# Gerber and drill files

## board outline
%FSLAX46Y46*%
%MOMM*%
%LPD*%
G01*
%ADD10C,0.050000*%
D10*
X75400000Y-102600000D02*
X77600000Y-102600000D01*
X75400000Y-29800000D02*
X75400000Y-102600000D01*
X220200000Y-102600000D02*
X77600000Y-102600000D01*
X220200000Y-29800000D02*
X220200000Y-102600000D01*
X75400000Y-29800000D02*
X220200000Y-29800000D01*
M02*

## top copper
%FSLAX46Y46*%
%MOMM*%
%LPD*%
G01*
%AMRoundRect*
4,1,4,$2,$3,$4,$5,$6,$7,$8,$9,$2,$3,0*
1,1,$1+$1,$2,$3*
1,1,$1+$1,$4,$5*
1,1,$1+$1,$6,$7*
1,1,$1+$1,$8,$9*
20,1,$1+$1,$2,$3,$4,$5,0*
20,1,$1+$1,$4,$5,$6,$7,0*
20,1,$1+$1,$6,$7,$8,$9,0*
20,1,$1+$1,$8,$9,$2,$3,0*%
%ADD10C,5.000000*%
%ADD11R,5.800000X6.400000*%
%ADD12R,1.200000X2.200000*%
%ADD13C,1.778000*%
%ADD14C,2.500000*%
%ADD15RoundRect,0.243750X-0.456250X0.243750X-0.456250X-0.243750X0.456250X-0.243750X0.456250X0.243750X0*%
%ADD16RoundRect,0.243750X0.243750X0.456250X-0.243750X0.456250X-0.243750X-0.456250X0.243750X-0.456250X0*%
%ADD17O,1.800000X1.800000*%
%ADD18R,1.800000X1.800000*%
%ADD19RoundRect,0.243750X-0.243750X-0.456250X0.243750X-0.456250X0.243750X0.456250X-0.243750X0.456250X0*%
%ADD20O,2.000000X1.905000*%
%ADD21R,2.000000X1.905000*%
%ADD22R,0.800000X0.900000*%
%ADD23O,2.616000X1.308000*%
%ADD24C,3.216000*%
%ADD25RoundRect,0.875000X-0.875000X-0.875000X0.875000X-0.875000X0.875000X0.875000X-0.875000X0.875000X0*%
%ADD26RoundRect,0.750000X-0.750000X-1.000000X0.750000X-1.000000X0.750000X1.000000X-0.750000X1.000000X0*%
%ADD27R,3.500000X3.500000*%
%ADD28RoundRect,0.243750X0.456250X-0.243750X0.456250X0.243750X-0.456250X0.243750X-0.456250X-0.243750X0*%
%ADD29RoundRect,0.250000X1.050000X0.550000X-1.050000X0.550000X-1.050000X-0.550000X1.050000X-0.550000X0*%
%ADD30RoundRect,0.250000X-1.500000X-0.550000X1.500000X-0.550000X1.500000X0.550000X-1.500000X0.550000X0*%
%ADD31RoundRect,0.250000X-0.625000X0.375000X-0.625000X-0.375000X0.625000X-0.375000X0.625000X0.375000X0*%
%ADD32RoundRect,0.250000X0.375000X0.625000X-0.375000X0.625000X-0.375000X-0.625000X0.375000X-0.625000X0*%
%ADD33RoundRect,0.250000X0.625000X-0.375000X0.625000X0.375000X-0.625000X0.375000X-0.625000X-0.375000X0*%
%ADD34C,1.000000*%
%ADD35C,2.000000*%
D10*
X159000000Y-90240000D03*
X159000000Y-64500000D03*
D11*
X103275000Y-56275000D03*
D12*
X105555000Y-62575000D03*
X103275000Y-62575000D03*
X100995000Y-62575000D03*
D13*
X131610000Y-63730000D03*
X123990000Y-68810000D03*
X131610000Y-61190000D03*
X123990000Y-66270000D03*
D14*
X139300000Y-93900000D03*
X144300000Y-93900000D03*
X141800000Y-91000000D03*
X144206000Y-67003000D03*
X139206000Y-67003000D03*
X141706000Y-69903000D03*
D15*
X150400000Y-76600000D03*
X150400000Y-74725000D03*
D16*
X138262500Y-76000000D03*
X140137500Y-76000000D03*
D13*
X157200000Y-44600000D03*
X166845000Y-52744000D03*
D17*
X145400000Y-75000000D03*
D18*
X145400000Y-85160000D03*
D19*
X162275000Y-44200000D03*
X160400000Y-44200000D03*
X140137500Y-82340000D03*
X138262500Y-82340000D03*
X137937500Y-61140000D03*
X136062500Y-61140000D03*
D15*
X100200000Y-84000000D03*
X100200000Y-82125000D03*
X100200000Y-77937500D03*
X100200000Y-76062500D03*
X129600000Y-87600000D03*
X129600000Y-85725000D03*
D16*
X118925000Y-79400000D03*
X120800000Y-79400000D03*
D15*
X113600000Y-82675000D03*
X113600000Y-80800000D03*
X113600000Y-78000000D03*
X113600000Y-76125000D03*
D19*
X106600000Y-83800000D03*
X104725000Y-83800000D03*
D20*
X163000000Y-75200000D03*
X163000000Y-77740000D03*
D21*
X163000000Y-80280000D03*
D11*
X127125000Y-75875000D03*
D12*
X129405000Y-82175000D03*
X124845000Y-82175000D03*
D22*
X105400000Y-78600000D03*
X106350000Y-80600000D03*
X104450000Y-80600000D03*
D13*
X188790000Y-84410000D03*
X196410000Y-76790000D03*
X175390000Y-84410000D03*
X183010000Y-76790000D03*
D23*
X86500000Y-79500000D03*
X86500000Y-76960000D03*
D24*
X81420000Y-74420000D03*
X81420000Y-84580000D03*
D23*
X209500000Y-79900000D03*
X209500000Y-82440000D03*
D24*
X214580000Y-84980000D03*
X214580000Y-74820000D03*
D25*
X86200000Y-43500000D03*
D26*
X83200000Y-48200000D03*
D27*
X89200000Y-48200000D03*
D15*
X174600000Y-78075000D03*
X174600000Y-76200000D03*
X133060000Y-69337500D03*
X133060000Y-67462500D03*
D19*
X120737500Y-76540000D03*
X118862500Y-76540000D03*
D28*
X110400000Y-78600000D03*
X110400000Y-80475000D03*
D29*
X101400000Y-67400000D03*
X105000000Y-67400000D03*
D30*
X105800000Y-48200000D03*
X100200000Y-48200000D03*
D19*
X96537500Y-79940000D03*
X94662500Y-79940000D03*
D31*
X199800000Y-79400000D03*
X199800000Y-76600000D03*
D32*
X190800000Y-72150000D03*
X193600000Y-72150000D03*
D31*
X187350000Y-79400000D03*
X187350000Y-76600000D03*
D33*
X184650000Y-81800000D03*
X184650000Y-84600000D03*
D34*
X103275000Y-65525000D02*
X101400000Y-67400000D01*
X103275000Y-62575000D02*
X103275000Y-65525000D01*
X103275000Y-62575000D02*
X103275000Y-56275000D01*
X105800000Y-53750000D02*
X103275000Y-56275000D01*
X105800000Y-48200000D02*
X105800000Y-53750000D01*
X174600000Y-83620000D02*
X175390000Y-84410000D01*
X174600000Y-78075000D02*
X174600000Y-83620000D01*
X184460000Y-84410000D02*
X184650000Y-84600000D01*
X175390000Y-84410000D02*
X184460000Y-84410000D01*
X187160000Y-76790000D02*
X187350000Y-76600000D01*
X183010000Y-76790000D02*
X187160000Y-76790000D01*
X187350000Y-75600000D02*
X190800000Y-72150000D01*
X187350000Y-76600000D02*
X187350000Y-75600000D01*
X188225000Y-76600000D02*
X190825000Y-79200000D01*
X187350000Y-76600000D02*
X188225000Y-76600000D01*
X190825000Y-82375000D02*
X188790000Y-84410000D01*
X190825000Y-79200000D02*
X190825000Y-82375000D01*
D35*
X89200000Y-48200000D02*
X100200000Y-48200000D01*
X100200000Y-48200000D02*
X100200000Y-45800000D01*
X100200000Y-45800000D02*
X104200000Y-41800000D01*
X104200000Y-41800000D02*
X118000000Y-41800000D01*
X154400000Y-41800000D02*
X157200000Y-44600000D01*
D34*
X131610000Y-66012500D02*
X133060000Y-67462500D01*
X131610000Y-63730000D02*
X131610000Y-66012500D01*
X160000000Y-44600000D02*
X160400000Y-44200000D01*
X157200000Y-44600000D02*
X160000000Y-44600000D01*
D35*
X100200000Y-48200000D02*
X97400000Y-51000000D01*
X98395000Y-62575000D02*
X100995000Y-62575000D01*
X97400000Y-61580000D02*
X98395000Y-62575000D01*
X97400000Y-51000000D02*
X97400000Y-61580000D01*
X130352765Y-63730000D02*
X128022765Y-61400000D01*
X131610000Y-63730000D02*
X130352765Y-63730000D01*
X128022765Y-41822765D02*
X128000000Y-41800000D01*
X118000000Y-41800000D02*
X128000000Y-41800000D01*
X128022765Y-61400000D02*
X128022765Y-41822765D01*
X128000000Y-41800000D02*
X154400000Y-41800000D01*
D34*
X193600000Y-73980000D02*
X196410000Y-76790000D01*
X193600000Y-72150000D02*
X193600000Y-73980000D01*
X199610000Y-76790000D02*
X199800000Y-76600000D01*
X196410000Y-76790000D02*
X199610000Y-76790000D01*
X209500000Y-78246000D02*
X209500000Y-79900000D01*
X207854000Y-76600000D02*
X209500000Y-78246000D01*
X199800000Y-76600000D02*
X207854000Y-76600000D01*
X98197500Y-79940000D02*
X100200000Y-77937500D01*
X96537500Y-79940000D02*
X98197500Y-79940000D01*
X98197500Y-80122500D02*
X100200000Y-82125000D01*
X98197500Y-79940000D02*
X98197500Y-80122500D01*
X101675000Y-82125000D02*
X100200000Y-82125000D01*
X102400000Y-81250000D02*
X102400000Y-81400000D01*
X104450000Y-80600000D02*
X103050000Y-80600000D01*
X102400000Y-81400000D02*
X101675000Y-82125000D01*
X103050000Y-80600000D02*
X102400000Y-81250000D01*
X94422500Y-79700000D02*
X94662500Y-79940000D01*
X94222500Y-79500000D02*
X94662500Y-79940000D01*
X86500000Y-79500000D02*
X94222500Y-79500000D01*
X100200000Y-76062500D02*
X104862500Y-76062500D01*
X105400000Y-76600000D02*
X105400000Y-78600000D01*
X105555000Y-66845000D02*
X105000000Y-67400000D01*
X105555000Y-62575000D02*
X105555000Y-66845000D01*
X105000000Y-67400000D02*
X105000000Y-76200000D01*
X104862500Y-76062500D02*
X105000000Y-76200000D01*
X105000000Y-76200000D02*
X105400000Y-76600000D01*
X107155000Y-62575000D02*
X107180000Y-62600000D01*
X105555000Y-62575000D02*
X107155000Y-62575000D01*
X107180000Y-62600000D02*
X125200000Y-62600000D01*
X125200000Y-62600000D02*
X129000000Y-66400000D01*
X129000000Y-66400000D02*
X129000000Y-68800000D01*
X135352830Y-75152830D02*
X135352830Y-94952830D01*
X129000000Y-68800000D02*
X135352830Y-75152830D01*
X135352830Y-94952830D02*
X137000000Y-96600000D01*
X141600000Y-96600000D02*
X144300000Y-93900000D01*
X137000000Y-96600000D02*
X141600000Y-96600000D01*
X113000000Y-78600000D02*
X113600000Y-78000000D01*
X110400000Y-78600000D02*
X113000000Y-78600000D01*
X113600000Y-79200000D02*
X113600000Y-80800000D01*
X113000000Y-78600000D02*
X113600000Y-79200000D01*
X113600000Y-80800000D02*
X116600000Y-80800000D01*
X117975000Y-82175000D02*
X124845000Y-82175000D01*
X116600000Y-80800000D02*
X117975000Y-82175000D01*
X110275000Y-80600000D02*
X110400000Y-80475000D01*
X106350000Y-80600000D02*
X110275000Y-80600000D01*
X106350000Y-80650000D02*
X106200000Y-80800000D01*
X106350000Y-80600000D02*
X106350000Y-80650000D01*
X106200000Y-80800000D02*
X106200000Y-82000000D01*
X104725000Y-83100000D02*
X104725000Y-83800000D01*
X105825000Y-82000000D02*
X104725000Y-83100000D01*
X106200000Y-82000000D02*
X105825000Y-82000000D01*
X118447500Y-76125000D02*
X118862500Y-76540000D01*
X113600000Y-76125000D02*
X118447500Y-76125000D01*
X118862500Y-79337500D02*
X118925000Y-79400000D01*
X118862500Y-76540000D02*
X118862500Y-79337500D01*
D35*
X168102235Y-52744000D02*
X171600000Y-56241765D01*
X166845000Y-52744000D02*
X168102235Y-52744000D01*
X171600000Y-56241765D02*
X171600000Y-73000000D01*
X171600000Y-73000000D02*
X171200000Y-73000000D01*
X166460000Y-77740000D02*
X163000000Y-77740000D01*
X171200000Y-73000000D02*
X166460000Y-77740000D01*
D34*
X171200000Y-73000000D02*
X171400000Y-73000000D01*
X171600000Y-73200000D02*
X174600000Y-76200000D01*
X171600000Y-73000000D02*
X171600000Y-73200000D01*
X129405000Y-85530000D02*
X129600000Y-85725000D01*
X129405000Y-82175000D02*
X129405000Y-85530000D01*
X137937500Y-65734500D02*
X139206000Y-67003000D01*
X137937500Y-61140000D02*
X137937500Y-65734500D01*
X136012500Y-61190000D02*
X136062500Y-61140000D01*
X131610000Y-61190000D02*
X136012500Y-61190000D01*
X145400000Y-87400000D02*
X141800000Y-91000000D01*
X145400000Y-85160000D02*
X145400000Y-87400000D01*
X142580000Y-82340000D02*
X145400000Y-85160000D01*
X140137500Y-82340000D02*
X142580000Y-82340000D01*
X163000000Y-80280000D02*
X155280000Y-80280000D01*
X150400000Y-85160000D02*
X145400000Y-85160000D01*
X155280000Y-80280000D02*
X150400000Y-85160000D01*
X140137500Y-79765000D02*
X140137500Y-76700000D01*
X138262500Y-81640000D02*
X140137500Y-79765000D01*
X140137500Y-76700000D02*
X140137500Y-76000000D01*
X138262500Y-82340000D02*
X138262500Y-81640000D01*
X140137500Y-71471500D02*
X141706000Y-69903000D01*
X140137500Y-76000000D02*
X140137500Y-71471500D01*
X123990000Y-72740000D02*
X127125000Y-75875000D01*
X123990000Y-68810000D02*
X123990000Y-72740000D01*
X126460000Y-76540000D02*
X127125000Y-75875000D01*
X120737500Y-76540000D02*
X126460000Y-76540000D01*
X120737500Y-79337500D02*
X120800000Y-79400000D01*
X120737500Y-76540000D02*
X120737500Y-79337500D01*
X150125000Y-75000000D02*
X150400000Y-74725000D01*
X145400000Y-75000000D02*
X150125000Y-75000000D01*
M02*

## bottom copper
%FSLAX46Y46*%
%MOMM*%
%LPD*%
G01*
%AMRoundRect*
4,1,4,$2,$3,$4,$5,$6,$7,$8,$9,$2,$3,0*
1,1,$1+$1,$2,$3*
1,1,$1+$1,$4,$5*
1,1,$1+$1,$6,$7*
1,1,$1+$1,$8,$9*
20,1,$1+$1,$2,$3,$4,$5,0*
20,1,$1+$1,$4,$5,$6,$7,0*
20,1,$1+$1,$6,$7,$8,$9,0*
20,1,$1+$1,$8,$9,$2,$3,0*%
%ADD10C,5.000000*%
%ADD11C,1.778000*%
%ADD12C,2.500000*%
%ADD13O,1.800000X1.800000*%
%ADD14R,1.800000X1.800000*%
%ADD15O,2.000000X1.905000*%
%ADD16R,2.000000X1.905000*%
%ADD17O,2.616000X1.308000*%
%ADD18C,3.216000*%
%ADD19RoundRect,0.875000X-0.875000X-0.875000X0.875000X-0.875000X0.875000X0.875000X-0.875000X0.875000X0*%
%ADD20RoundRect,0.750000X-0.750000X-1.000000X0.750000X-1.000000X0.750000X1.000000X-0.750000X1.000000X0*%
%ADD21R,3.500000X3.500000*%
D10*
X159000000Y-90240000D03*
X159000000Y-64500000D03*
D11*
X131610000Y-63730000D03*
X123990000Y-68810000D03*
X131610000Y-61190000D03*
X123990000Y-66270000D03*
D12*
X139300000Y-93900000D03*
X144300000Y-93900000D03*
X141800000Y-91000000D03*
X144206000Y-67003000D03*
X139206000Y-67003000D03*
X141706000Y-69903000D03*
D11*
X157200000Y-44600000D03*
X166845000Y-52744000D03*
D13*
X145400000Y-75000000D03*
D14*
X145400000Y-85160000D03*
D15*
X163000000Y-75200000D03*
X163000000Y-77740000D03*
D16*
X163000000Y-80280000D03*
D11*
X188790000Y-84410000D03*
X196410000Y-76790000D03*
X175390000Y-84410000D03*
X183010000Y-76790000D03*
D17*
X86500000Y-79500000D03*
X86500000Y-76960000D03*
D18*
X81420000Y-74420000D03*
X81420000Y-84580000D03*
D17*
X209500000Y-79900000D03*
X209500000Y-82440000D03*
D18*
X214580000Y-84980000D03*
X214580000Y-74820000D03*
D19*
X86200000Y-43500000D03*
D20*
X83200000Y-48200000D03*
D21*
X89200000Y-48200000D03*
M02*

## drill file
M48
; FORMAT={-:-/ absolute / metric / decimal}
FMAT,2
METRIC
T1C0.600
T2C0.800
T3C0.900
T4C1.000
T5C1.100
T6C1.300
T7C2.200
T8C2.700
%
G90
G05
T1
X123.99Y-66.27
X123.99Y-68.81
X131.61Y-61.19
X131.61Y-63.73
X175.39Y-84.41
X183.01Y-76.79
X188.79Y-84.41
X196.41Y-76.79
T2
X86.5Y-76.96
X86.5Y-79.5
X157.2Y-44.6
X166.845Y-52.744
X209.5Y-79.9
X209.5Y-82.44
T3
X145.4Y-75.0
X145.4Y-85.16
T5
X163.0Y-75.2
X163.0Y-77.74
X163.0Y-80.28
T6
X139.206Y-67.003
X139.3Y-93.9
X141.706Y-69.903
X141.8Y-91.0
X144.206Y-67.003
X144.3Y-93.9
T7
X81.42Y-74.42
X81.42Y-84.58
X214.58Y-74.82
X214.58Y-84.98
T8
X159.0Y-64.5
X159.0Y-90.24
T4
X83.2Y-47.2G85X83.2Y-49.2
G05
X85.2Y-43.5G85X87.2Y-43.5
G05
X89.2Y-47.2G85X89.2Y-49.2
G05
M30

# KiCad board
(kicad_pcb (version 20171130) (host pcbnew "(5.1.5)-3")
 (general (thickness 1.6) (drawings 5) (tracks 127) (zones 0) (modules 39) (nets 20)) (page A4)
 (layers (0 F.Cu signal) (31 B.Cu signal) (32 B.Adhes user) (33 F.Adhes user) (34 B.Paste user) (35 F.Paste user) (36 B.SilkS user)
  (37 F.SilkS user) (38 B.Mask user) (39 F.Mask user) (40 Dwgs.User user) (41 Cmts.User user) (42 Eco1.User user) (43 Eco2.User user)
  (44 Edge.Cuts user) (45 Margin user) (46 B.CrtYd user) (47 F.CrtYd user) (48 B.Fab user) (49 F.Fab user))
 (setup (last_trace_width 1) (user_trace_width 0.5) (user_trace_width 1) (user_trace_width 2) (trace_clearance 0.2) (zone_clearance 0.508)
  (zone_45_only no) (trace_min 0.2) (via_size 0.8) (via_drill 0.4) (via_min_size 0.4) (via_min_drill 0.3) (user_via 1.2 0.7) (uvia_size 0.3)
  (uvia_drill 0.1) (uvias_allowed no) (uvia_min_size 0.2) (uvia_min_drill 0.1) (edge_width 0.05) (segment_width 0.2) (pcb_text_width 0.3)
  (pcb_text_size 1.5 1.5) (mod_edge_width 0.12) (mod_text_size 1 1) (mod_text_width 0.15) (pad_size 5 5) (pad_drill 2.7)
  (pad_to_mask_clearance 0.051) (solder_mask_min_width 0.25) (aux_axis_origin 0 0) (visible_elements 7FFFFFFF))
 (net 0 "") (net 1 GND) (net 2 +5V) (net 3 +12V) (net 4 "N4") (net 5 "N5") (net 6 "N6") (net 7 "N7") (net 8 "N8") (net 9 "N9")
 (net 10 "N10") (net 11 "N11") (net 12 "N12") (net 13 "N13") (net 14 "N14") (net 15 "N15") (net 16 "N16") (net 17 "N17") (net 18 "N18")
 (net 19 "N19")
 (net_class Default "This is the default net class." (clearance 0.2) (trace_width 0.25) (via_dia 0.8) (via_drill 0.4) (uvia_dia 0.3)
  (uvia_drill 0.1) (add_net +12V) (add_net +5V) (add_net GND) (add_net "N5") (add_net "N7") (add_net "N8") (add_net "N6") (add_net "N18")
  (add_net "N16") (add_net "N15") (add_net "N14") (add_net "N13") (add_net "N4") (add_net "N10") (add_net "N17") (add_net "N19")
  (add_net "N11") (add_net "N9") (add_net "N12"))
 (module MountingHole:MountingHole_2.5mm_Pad (layer F.Cu) (at 159 90.24)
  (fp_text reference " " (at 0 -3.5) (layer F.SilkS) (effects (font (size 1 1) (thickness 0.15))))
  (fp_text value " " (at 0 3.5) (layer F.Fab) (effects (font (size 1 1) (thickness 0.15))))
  (pad 1 thru_hole circle (at 0 0) (size 5 5) (drill 2.7) (layers *.Cu *.Mask)))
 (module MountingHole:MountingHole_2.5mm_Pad (layer F.Cu) (at 159 64.5)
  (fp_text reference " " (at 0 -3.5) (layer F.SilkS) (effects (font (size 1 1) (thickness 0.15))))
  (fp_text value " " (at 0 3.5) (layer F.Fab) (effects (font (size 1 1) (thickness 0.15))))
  (pad 1 thru_hole circle (at 0 0) (size 5 5) (drill 2.7) (layers *.Cu *.Mask)))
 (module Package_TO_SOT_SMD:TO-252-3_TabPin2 (layer F.Cu) (at 103.275 58.375 90)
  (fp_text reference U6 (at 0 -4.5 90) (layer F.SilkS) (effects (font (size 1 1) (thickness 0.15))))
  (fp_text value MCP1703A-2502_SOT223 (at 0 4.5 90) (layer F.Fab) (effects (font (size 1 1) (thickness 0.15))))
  (pad "" smd rect (at 0.425 1.525 90) (size 3.05 2.75) (layers F.Paste))
  (pad "" smd rect (at 3.775 -1.525 90) (size 3.05 2.75) (layers F.Paste))
  (pad "" smd rect (at 0.425 -1.525 90) (size 3.05 2.75) (layers F.Paste))
  (pad "" smd rect (at 3.775 1.525 90) (size 3.05 2.75) (layers F.Paste))
  (pad 2 smd rect (at 2.1 0 90) (size 6.4 5.8) (layers F.Cu F.Mask) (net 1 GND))
  (pad 3 smd rect (at -4.2 2.28 90) (size 2.2 1.2) (layers F.Cu F.Paste F.Mask) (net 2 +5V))
  (pad 2 smd rect (at -4.2 0 90) (size 2.2 1.2) (layers F.Cu F.Paste F.Mask) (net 1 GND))
  (pad 1 smd rect (at -4.2 -2.28 90) (size 2.2 1.2) (layers F.Cu F.Paste F.Mask) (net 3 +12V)))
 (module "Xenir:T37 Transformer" (layer F.Cu) (at 127.8 58)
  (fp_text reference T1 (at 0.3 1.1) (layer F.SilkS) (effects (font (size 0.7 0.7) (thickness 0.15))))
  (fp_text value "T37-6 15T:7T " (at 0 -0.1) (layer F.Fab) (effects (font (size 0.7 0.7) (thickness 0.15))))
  (pad C1B thru_hole circle (at 3.81 5.73) (size 1.778 1.778) (drill 0.6) (layers *.Cu *.Mask) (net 3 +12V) (solder_mask_margin 0.1016))
  (pad C1A thru_hole circle (at -3.81 10.81) (size 1.778 1.778) (drill 0.6) (layers *.Cu *.Mask) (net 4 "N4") (solder_mask_margin 0.1016))
  (pad C2B thru_hole circle (at 3.81 3.19) (size 1.778 1.778) (drill 0.6) (layers *.Cu *.Mask) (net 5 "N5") (solder_mask_margin 0.1016))
  (pad C2A thru_hole circle (at -3.81 8.27) (size 1.778 1.778) (drill 0.6) (layers *.Cu *.Mask) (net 1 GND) (solder_mask_margin 0.1016)))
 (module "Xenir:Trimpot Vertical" (layer F.Cu) (at 136.506 92.503 90)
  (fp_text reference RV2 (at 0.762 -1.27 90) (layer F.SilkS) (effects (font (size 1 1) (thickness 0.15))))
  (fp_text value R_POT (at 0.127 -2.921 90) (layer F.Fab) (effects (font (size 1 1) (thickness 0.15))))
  (pad 1 thru_hole circle (at -1.397 2.794 90) (size 2.5 2.5) (drill 1.3) (layers *.Cu *.Mask) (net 1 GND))
  (pad 3 thru_hole circle (at -1.397 7.794 90) (size 2.5 2.5) (drill 1.3) (layers *.Cu *.Mask) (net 2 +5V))
  (pad 2 thru_hole circle (at 1.503 5.294 90) (size 2.5 2.5) (drill 1.3) (layers *.Cu *.Mask) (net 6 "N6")))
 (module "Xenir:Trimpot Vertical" (layer F.Cu) (at 147 68.4 270)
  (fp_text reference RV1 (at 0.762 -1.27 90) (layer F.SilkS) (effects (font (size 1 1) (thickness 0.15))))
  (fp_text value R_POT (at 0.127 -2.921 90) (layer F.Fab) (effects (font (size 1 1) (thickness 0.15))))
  (pad 1 thru_hole circle (at -1.397 2.794 270) (size 2.5 2.5) (drill 1.3) (layers *.Cu *.Mask) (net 1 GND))
  (pad 3 thru_hole circle (at -1.397 7.794 270) (size 2.5 2.5) (drill 1.3) (layers *.Cu *.Mask) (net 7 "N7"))
  (pad 2 thru_hole circle (at 1.503 5.294 270) (size 2.5 2.5) (drill 1.3) (layers *.Cu *.Mask) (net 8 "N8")))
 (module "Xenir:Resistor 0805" (layer F.Cu) (at 152.94 75.6625 270)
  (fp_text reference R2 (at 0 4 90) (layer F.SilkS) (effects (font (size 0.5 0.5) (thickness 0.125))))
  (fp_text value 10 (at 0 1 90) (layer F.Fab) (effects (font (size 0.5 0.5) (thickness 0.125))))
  (pad 2 smd roundrect (at 0.9375 2.54 270) (size 0.975 1.4) (layers F.Cu F.Paste F.Mask) (roundrect_rratio 0.25) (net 1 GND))
  (pad 1 smd roundrect (at -0.9375 2.54 270) (size 0.975 1.4) (layers F.Cu F.Paste F.Mask) (roundrect_rratio 0.25) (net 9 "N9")))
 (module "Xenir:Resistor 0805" (layer F.Cu) (at 139.2 78.54 180)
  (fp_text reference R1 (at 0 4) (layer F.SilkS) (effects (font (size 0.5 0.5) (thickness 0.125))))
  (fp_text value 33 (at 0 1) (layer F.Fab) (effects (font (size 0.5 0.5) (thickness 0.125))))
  (pad 2 smd roundrect (at 0.9375 2.54 180) (size 0.975 1.4) (layers F.Cu F.Paste F.Mask) (roundrect_rratio 0.25) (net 1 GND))
  (pad 1 smd roundrect (at -0.9375 2.54 180) (size 0.975 1.4) (layers F.Cu F.Paste F.Mask) (roundrect_rratio 0.25) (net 8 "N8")))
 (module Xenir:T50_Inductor (layer F.Cu) (at 170.789 48.41 270)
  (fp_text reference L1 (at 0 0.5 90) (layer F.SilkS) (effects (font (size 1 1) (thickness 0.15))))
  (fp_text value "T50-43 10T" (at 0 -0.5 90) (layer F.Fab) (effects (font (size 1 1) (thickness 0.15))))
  (pad 1 thru_hole circle (at -3.81 13.589 270) (size 1.778 1.778) (drill 0.8) (layers *.Cu *.Mask) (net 3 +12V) (solder_mask_margin 0.1016))
  (pad 2 thru_hole circle (at 4.334 3.944 270) (size 1.778 1.778) (drill 0.8) (layers *.Cu *.Mask) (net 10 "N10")
   (solder_mask_margin 0.1016)))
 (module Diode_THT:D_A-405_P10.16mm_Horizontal (layer F.Cu) (at 145.4 85.16 90)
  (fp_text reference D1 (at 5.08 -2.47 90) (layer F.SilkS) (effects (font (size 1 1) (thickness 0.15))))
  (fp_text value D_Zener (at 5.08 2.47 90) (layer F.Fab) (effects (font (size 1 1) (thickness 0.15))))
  (pad 2 thru_hole oval (at 10.16 0 90) (size 1.8 1.8) (drill 0.9) (layers *.Cu *.Mask) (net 9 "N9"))
  (pad 1 thru_hole rect (at 0 0 90) (size 1.8 1.8) (drill 0.9) (layers *.Cu *.Mask) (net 6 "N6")))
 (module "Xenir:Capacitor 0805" (layer F.Cu) (at 161.3375 41.66)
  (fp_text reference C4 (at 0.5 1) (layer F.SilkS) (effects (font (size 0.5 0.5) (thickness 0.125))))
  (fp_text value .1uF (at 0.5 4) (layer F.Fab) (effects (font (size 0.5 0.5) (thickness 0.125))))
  (pad 2 smd roundrect (at 0.9375 2.54) (size 0.975 1.4) (layers F.Cu F.Paste F.Mask) (roundrect_rratio 0.25) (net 1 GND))
  (pad 1 smd roundrect (at -0.9375 2.54) (size 0.975 1.4) (layers F.Cu F.Paste F.Mask) (roundrect_rratio 0.25) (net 3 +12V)))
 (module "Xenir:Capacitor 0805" (layer F.Cu) (at 139.2 79.8)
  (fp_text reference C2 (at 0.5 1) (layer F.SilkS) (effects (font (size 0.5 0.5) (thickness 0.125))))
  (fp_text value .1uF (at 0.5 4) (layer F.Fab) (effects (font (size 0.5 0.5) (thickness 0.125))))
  (pad 2 smd roundrect (at 0.9375 2.54) (size 0.975 1.4) (layers F.Cu F.Paste F.Mask) (roundrect_rratio 0.25) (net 6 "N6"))
  (pad 1 smd roundrect (at -0.9375 2.54) (size 0.975 1.4) (layers F.Cu F.Paste F.Mask) (roundrect_rratio 0.25) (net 8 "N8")))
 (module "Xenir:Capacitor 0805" (layer F.Cu) (at 137 58.6)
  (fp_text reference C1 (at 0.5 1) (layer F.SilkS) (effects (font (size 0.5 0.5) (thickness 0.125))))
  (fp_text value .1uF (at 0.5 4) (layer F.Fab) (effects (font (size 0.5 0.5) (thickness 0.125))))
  (pad 2 smd roundrect (at 0.9375 2.54) (size 0.975 1.4) (layers F.Cu F.Paste F.Mask) (roundrect_rratio 0.25) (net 7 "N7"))
  (pad 1 smd roundrect (at -0.9375 2.54) (size 0.975 1.4) (layers F.Cu F.Paste F.Mask) (roundrect_rratio 0.25) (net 5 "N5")))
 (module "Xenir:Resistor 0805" (layer F.Cu) (at 102.74 83.0625 270)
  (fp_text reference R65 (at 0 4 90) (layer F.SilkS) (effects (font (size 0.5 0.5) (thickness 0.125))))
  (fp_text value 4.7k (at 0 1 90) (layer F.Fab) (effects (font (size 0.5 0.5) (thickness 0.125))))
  (pad 2 smd roundrect (at 0.9375 2.54 270) (size 0.975 1.4) (layers F.Cu F.Paste F.Mask) (roundrect_rratio 0.25) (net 1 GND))
  (pad 1 smd roundrect (at -0.9375 2.54 270) (size 0.975 1.4) (layers F.Cu F.Paste F.Mask) (roundrect_rratio 0.25) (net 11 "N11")))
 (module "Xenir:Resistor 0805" (layer F.Cu) (at 102.74 77 270)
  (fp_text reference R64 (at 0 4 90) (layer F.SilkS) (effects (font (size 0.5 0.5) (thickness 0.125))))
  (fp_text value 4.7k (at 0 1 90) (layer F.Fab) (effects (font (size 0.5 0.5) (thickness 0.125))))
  (pad 2 smd roundrect (at 0.9375 2.54 270) (size 0.975 1.4) (layers F.Cu F.Paste F.Mask) (roundrect_rratio 0.25) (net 11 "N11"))
  (pad 1 smd roundrect (at -0.9375 2.54 270) (size 0.975 1.4) (layers F.Cu F.Paste F.Mask) (roundrect_rratio 0.25) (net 2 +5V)))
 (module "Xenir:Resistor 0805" (layer F.Cu) (at 132.14 86.6625 270)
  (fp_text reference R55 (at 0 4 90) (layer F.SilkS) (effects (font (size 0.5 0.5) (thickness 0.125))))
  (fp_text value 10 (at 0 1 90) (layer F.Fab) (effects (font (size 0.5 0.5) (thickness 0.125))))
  (pad 2 smd roundrect (at 0.9375 2.54 270) (size 0.975 1.4) (layers F.Cu F.Paste F.Mask) (roundrect_rratio 0.25) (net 1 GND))
  (pad 1 smd roundrect (at -0.9375 2.54 270) (size 0.975 1.4) (layers F.Cu F.Paste F.Mask) (roundrect_rratio 0.25) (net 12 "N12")))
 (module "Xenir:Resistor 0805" (layer F.Cu) (at 119.8625 81.94 180)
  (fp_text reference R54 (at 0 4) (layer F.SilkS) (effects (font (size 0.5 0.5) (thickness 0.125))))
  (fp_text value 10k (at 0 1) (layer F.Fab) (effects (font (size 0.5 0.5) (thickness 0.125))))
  (pad 2 smd roundrect (at 0.9375 2.54 180) (size 0.975 1.4) (layers F.Cu F.Paste F.Mask) (roundrect_rratio 0.25) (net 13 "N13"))
  (pad 1 smd roundrect (at -0.9375 2.54 180) (size 0.975 1.4) (layers F.Cu F.Paste F.Mask) (roundrect_rratio 0.25) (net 4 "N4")))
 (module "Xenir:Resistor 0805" (layer F.Cu) (at 116.14 81.7375 270)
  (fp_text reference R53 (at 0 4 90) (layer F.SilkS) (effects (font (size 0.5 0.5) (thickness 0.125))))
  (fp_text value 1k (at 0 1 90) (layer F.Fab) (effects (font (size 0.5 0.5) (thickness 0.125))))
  (pad 2 smd roundrect (at 0.9375 2.54 270) (size 0.975 1.4) (layers F.Cu F.Paste F.Mask) (roundrect_rratio 0.25) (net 1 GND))
  (pad 1 smd roundrect (at -0.9375 2.54 270) (size 0.975 1.4) (layers F.Cu F.Paste F.Mask) (roundrect_rratio 0.25) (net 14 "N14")))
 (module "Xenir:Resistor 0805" (layer F.Cu) (at 116.14 77.0625 270)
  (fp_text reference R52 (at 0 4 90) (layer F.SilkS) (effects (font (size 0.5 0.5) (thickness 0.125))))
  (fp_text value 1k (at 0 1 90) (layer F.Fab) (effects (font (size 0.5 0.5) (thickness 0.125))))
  (pad 2 smd roundrect (at 0.9375 2.54 270) (size 0.975 1.4) (layers F.Cu F.Paste F.Mask) (roundrect_rratio 0.25) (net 14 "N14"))
  (pad 1 smd roundrect (at -0.9375 2.54 270) (size 0.975 1.4) (layers F.Cu F.Paste F.Mask) (roundrect_rratio 0.25) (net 13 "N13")))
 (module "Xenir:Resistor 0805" (layer F.Cu) (at 105.6625 81.26)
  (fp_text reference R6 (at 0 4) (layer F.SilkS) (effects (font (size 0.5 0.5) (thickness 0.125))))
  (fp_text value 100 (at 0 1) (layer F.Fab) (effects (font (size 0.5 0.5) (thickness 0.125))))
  (pad 2 smd roundrect (at 0.9375 2.54) (size 0.975 1.4) (layers F.Cu F.Paste F.Mask) (roundrect_rratio 0.25) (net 1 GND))
  (pad 1 smd roundrect (at -0.9375 2.54) (size 0.975 1.4) (layers F.Cu F.Paste F.Mask) (roundrect_rratio 0.25) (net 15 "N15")))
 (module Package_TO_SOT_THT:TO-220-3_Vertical (layer F.Cu) (at 163 80.28 90)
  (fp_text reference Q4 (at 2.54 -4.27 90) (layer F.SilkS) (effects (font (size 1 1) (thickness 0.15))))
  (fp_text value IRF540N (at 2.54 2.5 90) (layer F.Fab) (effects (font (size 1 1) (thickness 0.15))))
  (pad 3 thru_hole oval (at 5.08 0 90) (size 1.905 2) (drill 1.1) (layers *.Cu *.Mask) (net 1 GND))
  (pad 2 thru_hole oval (at 2.54 0 90) (size 1.905 2) (drill 1.1) (layers *.Cu *.Mask) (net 10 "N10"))
  (pad 1 thru_hole rect (at 0 0 90) (size 1.905 2) (drill 1.1) (layers *.Cu *.Mask) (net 6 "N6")))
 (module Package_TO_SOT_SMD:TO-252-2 (layer F.Cu) (at 127.125 77.975 90)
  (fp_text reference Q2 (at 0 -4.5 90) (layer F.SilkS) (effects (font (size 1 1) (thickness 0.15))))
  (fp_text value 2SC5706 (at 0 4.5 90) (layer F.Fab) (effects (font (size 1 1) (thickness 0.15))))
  (pad "" smd rect (at 0.425 1.525 90) (size 3.05 2.75) (layers F.Paste))
  (pad "" smd rect (at 3.775 -1.525 90) (size 3.05 2.75) (layers F.Paste))
  (pad "" smd rect (at 0.425 -1.525 90) (size 3.05 2.75) (layers F.Paste))
  (pad "" smd rect (at 3.775 1.525 90) (size 3.05 2.75) (layers F.Paste))
  (pad 2 smd rect (at 2.1 0 90) (size 6.4 5.8) (layers F.Cu F.Mask) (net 4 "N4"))
  (pad 3 smd rect (at -4.2 2.28 90) (size 2.2 1.2) (layers F.Cu F.Paste F.Mask) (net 12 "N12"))
  (pad 1 smd rect (at -4.2 -2.28 90) (size 2.2 1.2) (layers F.Cu F.Paste F.Mask) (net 14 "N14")))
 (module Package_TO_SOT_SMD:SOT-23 (layer F.Cu) (at 105.4 79.6 90)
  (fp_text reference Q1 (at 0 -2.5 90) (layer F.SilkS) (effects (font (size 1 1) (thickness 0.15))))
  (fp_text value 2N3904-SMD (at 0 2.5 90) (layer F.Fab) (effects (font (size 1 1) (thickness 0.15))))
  (pad 3 smd rect (at 1 0 90) (size 0.9 0.8) (layers F.Cu F.Paste F.Mask) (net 2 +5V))
  (pad 2 smd rect (at -1 0.95 90) (size 0.9 0.8) (layers F.Cu F.Paste F.Mask) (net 15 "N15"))
  (pad 1 smd rect (at -1 -0.95 90) (size 0.9 0.8) (layers F.Cu F.Paste F.Mask) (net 11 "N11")))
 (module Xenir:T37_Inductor (layer F.Cu) (at 192.6 73.6)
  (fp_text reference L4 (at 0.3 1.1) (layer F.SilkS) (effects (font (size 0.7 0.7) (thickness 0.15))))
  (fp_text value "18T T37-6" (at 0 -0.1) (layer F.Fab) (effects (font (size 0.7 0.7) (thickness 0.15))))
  (pad 1 thru_hole circle (at -3.81 10.81) (size 1.778 1.778) (drill 0.6) (layers *.Cu *.Mask) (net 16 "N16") (solder_mask_margin 0.1016))
  (pad 2 thru_hole circle (at 3.81 3.19) (size 1.778 1.778) (drill 0.6) (layers *.Cu *.Mask) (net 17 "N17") (solder_mask_margin 0.1016)))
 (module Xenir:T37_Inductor (layer F.Cu) (at 179.2 73.6)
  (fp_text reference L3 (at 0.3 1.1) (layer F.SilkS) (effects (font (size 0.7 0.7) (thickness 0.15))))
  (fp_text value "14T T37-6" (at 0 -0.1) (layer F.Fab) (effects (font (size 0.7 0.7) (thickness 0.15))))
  (pad 1 thru_hole circle (at -3.81 10.81) (size 1.778 1.778) (drill 0.6) (layers *.Cu *.Mask) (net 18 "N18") (solder_mask_margin 0.1016))
  (pad 2 thru_hole circle (at 3.81 3.19) (size 1.778 1.778) (drill 0.6) (layers *.Cu *.Mask) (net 16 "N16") (solder_mask_margin 0.1016)))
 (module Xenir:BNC (layer B.Cu) (at 82.6 79.6 270)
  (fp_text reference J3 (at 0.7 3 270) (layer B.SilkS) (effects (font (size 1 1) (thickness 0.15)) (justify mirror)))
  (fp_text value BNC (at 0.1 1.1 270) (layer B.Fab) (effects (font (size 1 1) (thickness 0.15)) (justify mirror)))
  (pad S thru_hole oval (at -0.1 -3.9 180) (size 2.616 1.308) (drill 0.8) (layers *.Cu *.Mask) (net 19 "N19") (solder_mask_margin 0.1016))
  (pad GND thru_hole oval (at -2.64 -3.9 180) (size 2.616 1.308) (drill 0.8) (layers *.Cu *.Mask) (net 1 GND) (solder_mask_margin 0.1016))
  (pad 3 thru_hole circle (at -5.18 1.18 270) (size 3.216 3.216) (drill 2.2) (layers *.Cu *.Mask) (solder_mask_margin 0.1016))
  (pad 4 thru_hole circle (at 4.98 1.18 270) (size 3.216 3.216) (drill 2.2) (layers *.Cu *.Mask) (solder_mask_margin 0.1016)))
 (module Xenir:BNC (layer B.Cu) (at 213.4 79.8 90)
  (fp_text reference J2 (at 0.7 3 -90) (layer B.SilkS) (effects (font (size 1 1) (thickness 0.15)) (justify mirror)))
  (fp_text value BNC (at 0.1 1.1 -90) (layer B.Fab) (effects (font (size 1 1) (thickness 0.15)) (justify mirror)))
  (pad S thru_hole oval (at -0.1 -3.9) (size 2.616 1.308) (drill 0.8) (layers *.Cu *.Mask) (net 17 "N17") (solder_mask_margin 0.1016))
  (pad GND thru_hole oval (at -2.64 -3.9) (size 2.616 1.308) (drill 0.8) (layers *.Cu *.Mask) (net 1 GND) (solder_mask_margin 0.1016))
  (pad 3 thru_hole circle (at -5.18 1.18 90) (size 3.216 3.216) (drill 2.2) (layers *.Cu *.Mask) (solder_mask_margin 0.1016))
  (pad 4 thru_hole circle (at 4.98 1.18 90) (size 3.216 3.216) (drill 2.2) (layers *.Cu *.Mask) (solder_mask_margin 0.1016)))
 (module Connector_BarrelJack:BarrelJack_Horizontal (layer B.Cu) (at 89.2 48.2)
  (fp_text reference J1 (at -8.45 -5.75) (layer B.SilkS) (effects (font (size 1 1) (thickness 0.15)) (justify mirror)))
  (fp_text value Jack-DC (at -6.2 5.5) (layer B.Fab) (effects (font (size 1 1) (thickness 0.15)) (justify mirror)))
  (pad 3 thru_hole roundrect (at -3 -4.7) (size 3.5 3.5) (drill oval 3 1) (layers *.Cu *.Mask) (roundrect_rratio 0.25))
  (pad 2 thru_hole roundrect (at -6 0) (size 3 3.5) (drill oval 1 3) (layers *.Cu *.Mask) (roundrect_rratio 0.25) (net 1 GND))
  (pad 1 thru_hole rect (at 0 0) (size 3.5 3.5) (drill oval 1 3) (layers *.Cu *.Mask) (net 3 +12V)))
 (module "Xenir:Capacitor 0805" (layer F.Cu) (at 177.14 77.1375 270)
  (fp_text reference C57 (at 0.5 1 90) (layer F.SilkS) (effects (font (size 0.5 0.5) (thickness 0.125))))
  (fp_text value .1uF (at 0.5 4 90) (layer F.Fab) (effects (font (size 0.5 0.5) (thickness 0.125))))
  (pad 2 smd roundrect (at 0.9375 2.54 270) (size 0.975 1.4) (layers F.Cu F.Paste F.Mask) (roundrect_rratio 0.25) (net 18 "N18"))
  (pad 1 smd roundrect (at -0.9375 2.54 270) (size 0.975 1.4) (layers F.Cu F.Paste F.Mask) (roundrect_rratio 0.25) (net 10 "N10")))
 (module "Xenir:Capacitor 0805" (layer F.Cu) (at 135.6 68.4 270)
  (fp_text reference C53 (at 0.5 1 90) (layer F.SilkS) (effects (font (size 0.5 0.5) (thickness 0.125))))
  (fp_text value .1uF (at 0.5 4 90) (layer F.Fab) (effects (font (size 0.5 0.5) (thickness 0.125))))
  (pad 2 smd roundrect (at 0.9375 2.54 270) (size 0.975 1.4) (layers F.Cu F.Paste F.Mask) (roundrect_rratio 0.25) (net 1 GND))
  (pad 1 smd roundrect (at -0.9375 2.54 270) (size 0.975 1.4) (layers F.Cu F.Paste F.Mask) (roundrect_rratio 0.25) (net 3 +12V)))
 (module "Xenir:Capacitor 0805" (layer F.Cu) (at 119.8 74)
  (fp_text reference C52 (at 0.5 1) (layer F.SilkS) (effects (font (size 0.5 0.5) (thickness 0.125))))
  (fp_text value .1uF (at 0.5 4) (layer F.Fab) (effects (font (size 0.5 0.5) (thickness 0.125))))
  (pad 2 smd roundrect (at 0.9375 2.54) (size 0.975 1.4) (layers F.Cu F.Paste F.Mask) (roundrect_rratio 0.25) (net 4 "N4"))
  (pad 1 smd roundrect (at -0.9375 2.54) (size 0.975 1.4) (layers F.Cu F.Paste F.Mask) (roundrect_rratio 0.25) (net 13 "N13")))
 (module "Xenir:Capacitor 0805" (layer F.Cu) (at 107.86 79.5375 90)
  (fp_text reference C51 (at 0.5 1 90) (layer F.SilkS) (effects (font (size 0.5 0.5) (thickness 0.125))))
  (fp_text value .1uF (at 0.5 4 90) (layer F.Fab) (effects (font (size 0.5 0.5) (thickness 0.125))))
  (pad 2 smd roundrect (at 0.9375 2.54 90) (size 0.975 1.4) (layers F.Cu F.Paste F.Mask) (roundrect_rratio 0.25) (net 14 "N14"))
  (pad 1 smd roundrect (at -0.9375 2.54 90) (size 0.975 1.4) (layers F.Cu F.Paste F.Mask) (roundrect_rratio 0.25) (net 15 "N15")))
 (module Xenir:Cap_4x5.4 (layer F.Cu) (at 103.2 67.9 180)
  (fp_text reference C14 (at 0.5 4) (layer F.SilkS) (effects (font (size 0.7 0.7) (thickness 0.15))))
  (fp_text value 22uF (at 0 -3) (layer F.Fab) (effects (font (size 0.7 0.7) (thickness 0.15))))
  (pad 2 smd roundrect (at 1.8 0.5 180) (size 2.6 1.6) (layers F.Cu F.Paste F.Mask) (roundrect_rratio 0.15625) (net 1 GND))
  (pad 1 smd roundrect (at -1.8 0.5 180) (size 2.6 1.6) (layers F.Cu F.Paste F.Mask) (roundrect_rratio 0.15625) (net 2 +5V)))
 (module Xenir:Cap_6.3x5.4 (layer F.Cu) (at 102.9 42.1)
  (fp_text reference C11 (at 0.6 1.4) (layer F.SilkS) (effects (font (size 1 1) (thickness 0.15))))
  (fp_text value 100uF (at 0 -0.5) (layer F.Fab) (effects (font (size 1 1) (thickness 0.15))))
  (pad 2 smd roundrect (at 2.9 6.1) (size 3.5 1.6) (layers F.Cu F.Paste F.Mask) (roundrect_rratio 0.15625) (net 1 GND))
  (pad 1 smd roundrect (at -2.7 6.1) (size 3.5 1.6) (layers F.Cu F.Paste F.Mask) (roundrect_rratio 0.15625) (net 3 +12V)))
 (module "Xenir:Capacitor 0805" (layer F.Cu) (at 95.6 77.4)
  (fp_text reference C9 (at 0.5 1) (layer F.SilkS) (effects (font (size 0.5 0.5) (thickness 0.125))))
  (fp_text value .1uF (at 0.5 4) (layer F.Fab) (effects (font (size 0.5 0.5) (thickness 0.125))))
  (pad 2 smd roundrect (at 0.9375 2.54) (size 0.975 1.4) (layers F.Cu F.Paste F.Mask) (roundrect_rratio 0.25) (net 11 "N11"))
  (pad 1 smd roundrect (at -0.9375 2.54) (size 0.975 1.4) (layers F.Cu F.Paste F.Mask) (roundrect_rratio 0.25) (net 19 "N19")))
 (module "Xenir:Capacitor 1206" (layer F.Cu) (at 202.05 78 270)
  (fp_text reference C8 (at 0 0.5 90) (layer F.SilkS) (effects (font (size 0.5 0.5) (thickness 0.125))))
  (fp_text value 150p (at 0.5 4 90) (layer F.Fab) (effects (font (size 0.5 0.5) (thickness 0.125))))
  (pad 2 smd roundrect (at 1.4 2.25 270) (size 1.25 1.75) (layers F.Cu F.Paste F.Mask) (roundrect_rratio 0.2) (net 1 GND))
  (pad 1 smd roundrect (at -1.4 2.25 270) (size 1.25 1.75) (layers F.Cu F.Paste F.Mask) (roundrect_rratio 0.2) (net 17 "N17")))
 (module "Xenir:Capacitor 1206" (layer F.Cu) (at 192.2 74.4 180)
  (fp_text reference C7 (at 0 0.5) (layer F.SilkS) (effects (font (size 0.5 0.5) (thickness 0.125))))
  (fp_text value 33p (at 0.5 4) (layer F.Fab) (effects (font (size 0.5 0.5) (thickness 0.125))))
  (pad 2 smd roundrect (at 1.4 2.25 180) (size 1.25 1.75) (layers F.Cu F.Paste F.Mask) (roundrect_rratio 0.2) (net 16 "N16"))
  (pad 1 smd roundrect (at -1.4 2.25 180) (size 1.25 1.75) (layers F.Cu F.Paste F.Mask) (roundrect_rratio 0.2) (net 17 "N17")))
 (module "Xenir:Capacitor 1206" (layer F.Cu) (at 189.6 78 270)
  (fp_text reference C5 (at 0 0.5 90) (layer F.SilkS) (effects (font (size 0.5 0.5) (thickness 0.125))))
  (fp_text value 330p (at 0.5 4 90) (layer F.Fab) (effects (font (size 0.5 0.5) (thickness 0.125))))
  (pad 2 smd roundrect (at 1.4 2.25 270) (size 1.25 1.75) (layers F.Cu F.Paste F.Mask) (roundrect_rratio 0.2) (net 1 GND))
  (pad 1 smd roundrect (at -1.4 2.25 270) (size 1.25 1.75) (layers F.Cu F.Paste F.Mask) (roundrect_rratio 0.2) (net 16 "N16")))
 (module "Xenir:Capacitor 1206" (layer F.Cu) (at 182.4 83.2 90)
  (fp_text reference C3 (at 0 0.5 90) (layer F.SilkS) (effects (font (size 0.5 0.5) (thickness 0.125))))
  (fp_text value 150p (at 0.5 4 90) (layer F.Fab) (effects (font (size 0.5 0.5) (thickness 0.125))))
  (pad 2 smd roundrect (at 1.4 2.25 90) (size 1.25 1.75) (layers F.Cu F.Paste F.Mask) (roundrect_rratio 0.2) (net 1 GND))
  (pad 1 smd roundrect (at -1.4 2.25 90) (size 1.25 1.75) (layers F.Cu F.Paste F.Mask) (roundrect_rratio 0.2) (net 18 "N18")))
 (gr_line (start 75.4 102.6) (end 77.6 102.6) (layer Edge.Cuts) (width 0.05))
 (gr_line (start 75.4 29.8) (end 75.4 102.6) (layer Edge.Cuts) (width 0.05))
 (gr_line (start 220.2 102.6) (end 77.6 102.6) (layer Edge.Cuts) (width 0.05))
 (gr_line (start 220.2 29.8) (end 220.2 102.6) (layer Edge.Cuts) (width 0.05))
 (gr_line (start 75.4 29.8) (end 220.2 29.8) (layer Edge.Cuts) (width 0.05))
 (segment (start 103.275 65.525) (end 101.4 67.4) (width 1) (layer F.Cu) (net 1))
 (segment (start 103.275 62.575) (end 103.275 65.525) (width 1) (layer F.Cu) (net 1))
 (segment (start 103.275 62.575) (end 103.275 56.275) (width 1) (layer F.Cu) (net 1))
 (segment (start 105.8 53.75) (end 103.275 56.275) (width 1) (layer F.Cu) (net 1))
 (segment (start 105.8 48.2) (end 105.8 53.75) (width 1) (layer F.Cu) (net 1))
 (segment (start 174.6 83.62) (end 175.39 84.41) (width 1) (layer F.Cu) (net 18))
 (segment (start 174.6 78.075) (end 174.6 83.62) (width 1) (layer F.Cu) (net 18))
 (segment (start 184.46 84.41) (end 184.65 84.6) (width 1) (layer F.Cu) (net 18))
 (segment (start 175.39 84.41) (end 184.46 84.41) (width 1) (layer F.Cu) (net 18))
 (segment (start 187.16 76.79) (end 187.35 76.6) (width 1) (layer F.Cu) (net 16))
 (segment (start 183.01 76.79) (end 187.16 76.79) (width 1) (layer F.Cu) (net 16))
 (segment (start 187.35 75.6) (end 190.8 72.15) (width 1) (layer F.Cu) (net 16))
 (segment (start 187.35 76.6) (end 187.35 75.6) (width 1) (layer F.Cu) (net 16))
 (segment (start 188.225 76.6) (end 190.825 79.2) (width 1) (layer F.Cu) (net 16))
 (segment (start 187.35 76.6) (end 188.225 76.6) (width 1) (layer F.Cu) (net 16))
 (segment (start 190.825 82.375) (end 188.79 84.41) (width 1) (layer F.Cu) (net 16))
 (segment (start 190.825 79.2) (end 190.825 82.375) (width 1) (layer F.Cu) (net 16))
 (segment (start 89.2 48.2) (end 100.2 48.2) (width 2) (layer F.Cu) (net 3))
 (segment (start 100.2 48.2) (end 100.2 45.8) (width 2) (layer F.Cu) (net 3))
 (segment (start 100.2 45.8) (end 104.2 41.8) (width 2) (layer F.Cu) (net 3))
 (segment (start 104.2 41.8) (end 118 41.8) (width 2) (layer F.Cu) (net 3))
 (segment (start 154.4 41.8) (end 157.2 44.6) (width 2) (layer F.Cu) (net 3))
 (segment (start 131.61 66.0125) (end 133.06 67.4625) (width 1) (layer F.Cu) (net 3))
 (segment (start 131.61 63.73) (end 131.61 66.0125) (width 1) (layer F.Cu) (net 3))
 (segment (start 160 44.6) (end 160.4 44.2) (width 1) (layer F.Cu) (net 3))
 (segment (start 157.2 44.6) (end 160 44.6) (width 1) (layer F.Cu) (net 3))
 (segment (start 100.2 48.2) (end 97.4 51) (width 2) (layer F.Cu) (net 3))
 (segment (start 98.395 62.575) (end 100.995 62.575) (width 2) (layer F.Cu) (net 3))
 (segment (start 97.4 61.58) (end 98.395 62.575) (width 2) (layer F.Cu) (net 3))
 (segment (start 97.4 51) (end 97.4 61.58) (width 2) (layer F.Cu) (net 3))
 (segment (start 130.352765 63.73) (end 128.022765 61.4) (width 2) (layer F.Cu) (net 3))
 (segment (start 131.61 63.73) (end 130.352765 63.73) (width 2) (layer F.Cu) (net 3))
 (segment (start 128.022765 41.822765) (end 128 41.8) (width 2) (layer F.Cu) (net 3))
 (segment (start 118 41.8) (end 128 41.8) (width 2) (layer F.Cu) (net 3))
 (segment (start 128.022765 61.4) (end 128.022765 41.822765) (width 2) (layer F.Cu) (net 3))
 (segment (start 128 41.8) (end 154.4 41.8) (width 2) (layer F.Cu) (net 3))
 (segment (start 193.6 73.98) (end 196.41 76.79) (width 1) (layer F.Cu) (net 17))
 (segment (start 193.6 72.15) (end 193.6 73.98) (width 1) (layer F.Cu) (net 17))
 (segment (start 199.61 76.79) (end 199.8 76.6) (width 1) (layer F.Cu) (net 17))
 (segment (start 196.41 76.79) (end 199.61 76.79) (width 1) (layer F.Cu) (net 17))
 (segment (start 209.5 78.246) (end 209.5 79.9) (width 1) (layer F.Cu) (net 17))
 (segment (start 207.854 76.6) (end 209.5 78.246) (width 1) (layer F.Cu) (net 17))
 (segment (start 199.8 76.6) (end 207.854 76.6) (width 1) (layer F.Cu) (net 17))
 (segment (start 98.1975 79.94) (end 100.2 77.9375) (width 1) (layer F.Cu) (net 11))
 (segment (start 96.5375 79.94) (end 98.1975 79.94) (width 1) (layer F.Cu) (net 11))
 (segment (start 98.1975 80.1225) (end 100.2 82.125) (width 1) (layer F.Cu) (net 11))
 (segment (start 98.1975 79.94) (end 98.1975 80.1225) (width 1) (layer F.Cu) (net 11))
 (segment (start 101.675 82.125) (end 100.2 82.125) (width 1) (layer F.Cu) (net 11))
 (segment (start 102.4 81.25) (end 102.4 81.4) (width 1) (layer F.Cu) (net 11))
 (segment (start 104.45 80.6) (end 103.05 80.6) (width 1) (layer F.Cu) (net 11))
 (segment (start 102.4 81.4) (end 101.675 82.125) (width 1) (layer F.Cu) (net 11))
 (segment (start 103.05 80.6) (end 102.4 81.25) (width 1) (layer F.Cu) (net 11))
 (segment (start 94.4225 79.7) (end 94.6625 79.94) (width 1) (layer F.Cu) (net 19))
 (segment (start 94.2225 79.5) (end 94.6625 79.94) (width 1) (layer F.Cu) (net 19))
 (segment (start 86.5 79.5) (end 94.2225 79.5) (width 1) (layer F.Cu) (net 19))
 (segment (start 100.2 76.0625) (end 104.8625 76.0625) (width 1) (layer F.Cu) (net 2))
 (segment (start 105.4 76.6) (end 105.4 78.6) (width 1) (layer F.Cu) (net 2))
 (segment (start 105.555 66.845) (end 105 67.4) (width 1) (layer F.Cu) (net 2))
 (segment (start 105.555 62.575) (end 105.555 66.845) (width 1) (layer F.Cu) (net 2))
 (segment (start 105 67.4) (end 105 76.2) (width 1) (layer F.Cu) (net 2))
 (segment (start 104.8625 76.0625) (end 105 76.2) (width 1) (layer F.Cu) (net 2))
 (segment (start 105 76.2) (end 105.4 76.6) (width 1) (layer F.Cu) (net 2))
 (segment (start 107.155 62.575) (end 107.18 62.6) (width 1) (layer F.Cu) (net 2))
 (segment (start 105.555 62.575) (end 107.155 62.575) (width 1) (layer F.Cu) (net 2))
 (segment (start 107.18 62.6) (end 125.2 62.6) (width 1) (layer F.Cu) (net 2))
 (segment (start 125.2 62.6) (end 129 66.4) (width 1) (layer F.Cu) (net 2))
 (segment (start 129 66.4) (end 129 68.8) (width 1) (layer F.Cu) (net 2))
 (segment (start 135.35283 75.15283) (end 135.35283 94.95283) (width 1) (layer F.Cu) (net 2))
 (segment (start 129 68.8) (end 135.35283 75.15283) (width 1) (layer F.Cu) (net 2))
 (segment (start 135.35283 94.95283) (end 137 96.6) (width 1) (layer F.Cu) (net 2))
 (segment (start 141.6 96.6) (end 144.3 93.9) (width 1) (layer F.Cu) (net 2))
 (segment (start 137 96.6) (end 141.6 96.6) (width 1) (layer F.Cu) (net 2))
 (segment (start 113 78.6) (end 113.6 78) (width 1) (layer F.Cu) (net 14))
 (segment (start 110.4 78.6) (end 113 78.6) (width 1) (layer F.Cu) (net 14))
 (segment (start 113.6 79.2) (end 113.6 80.8) (width 1) (layer F.Cu) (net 14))
 (segment (start 113 78.6) (end 113.6 79.2) (width 1) (layer F.Cu) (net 14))
 (segment (start 113.6 80.8) (end 116.6 80.8) (width 1) (layer F.Cu) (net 14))
 (segment (start 117.975 82.175) (end 124.845 82.175) (width 1) (layer F.Cu) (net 14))
 (segment (start 116.6 80.8) (end 117.975 82.175) (width 1) (layer F.Cu) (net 14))
 (segment (start 110.275 80.6) (end 110.4 80.475) (width 1) (layer F.Cu) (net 15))
 (segment (start 106.35 80.6) (end 110.275 80.6) (width 1) (layer F.Cu) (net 15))
 (segment (start 106.35 80.65) (end 106.2 80.8) (width 1) (layer F.Cu) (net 15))
 (segment (start 106.35 80.6) (end 106.35 80.65) (width 1) (layer F.Cu) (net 15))
 (segment (start 106.2 80.8) (end 106.2 82) (width 1) (layer F.Cu) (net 15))
 (segment (start 104.725 83.1) (end 104.725 83.8) (width 1) (layer F.Cu) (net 15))
 (segment (start 105.825 82) (end 104.725 83.1) (width 1) (layer F.Cu) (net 15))
 (segment (start 106.2 82) (end 105.825 82) (width 1) (layer F.Cu) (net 15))
 (segment (start 118.4475 76.125) (end 118.8625 76.54) (width 1) (layer F.Cu) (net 13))
 (segment (start 113.6 76.125) (end 118.4475 76.125) (width 1) (layer F.Cu) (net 13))
 (segment (start 118.8625 79.3375) (end 118.925 79.4) (width 1) (layer F.Cu) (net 13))
 (segment (start 118.8625 76.54) (end 118.8625 79.3375) (width 1) (layer F.Cu) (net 13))
 (segment (start 168.102235 52.744) (end 171.6 56.241765) (width 2) (layer F.Cu) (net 10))
 (segment (start 166.845 52.744) (end 168.102235 52.744) (width 2) (layer F.Cu) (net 10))
 (segment (start 171.6 56.241765) (end 171.6 73) (width 2) (layer F.Cu) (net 10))
 (segment (start 171.6 73) (end 171.2 73) (width 2) (layer F.Cu) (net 10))
 (segment (start 166.46 77.74) (end 163 77.74) (width 2) (layer F.Cu) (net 10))
 (segment (start 171.2 73) (end 166.46 77.74) (width 2) (layer F.Cu) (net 10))
 (segment (start 171.2 73) (end 171.4 73) (width 1) (layer F.Cu) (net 10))
 (segment (start 171.6 73.2) (end 174.6 76.2) (width 1) (layer F.Cu) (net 10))
 (segment (start 171.6 73) (end 171.6 73.2) (width 1) (layer F.Cu) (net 10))
 (segment (start 129.405 85.53) (end 129.6 85.725) (width 1) (layer F.Cu) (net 12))
 (segment (start 129.405 82.175) (end 129.405 85.53) (width 1) (layer F.Cu) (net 12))
 (segment (start 137.9375 65.7345) (end 139.206 67.003) (width 1) (layer F.Cu) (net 7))
 (segment (start 137.9375 61.14) (end 137.9375 65.7345) (width 1) (layer F.Cu) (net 7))
 (segment (start 136.0125 61.19) (end 136.0625 61.14) (width 1) (layer F.Cu) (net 5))
 (segment (start 131.61 61.19) (end 136.0125 61.19) (width 1) (layer F.Cu) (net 5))
 (segment (start 145.4 87.4) (end 141.8 91) (width 1) (layer F.Cu) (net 6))
 (segment (start 145.4 85.16) (end 145.4 87.4) (width 1) (layer F.Cu) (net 6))
 (segment (start 142.58 82.34) (end 145.4 85.16) (width 1) (layer F.Cu) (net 6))
 (segment (start 140.1375 82.34) (end 142.58 82.34) (width 1) (layer F.Cu) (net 6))
 (segment (start 163 80.28) (end 155.28 80.28) (width 1) (layer F.Cu) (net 6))
 (segment (start 150.4 85.16) (end 145.4 85.16) (width 1) (layer F.Cu) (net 6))
 (segment (start 155.28 80.28) (end 150.4 85.16) (width 1) (layer F.Cu) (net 6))
 (segment (start 140.1375 79.765) (end 140.1375 76.7) (width 1) (layer F.Cu) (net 8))
 (segment (start 138.2625 81.64) (end 140.1375 79.765) (width 1) (layer F.Cu) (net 8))
 (segment (start 140.1375 76.7) (end 140.1375 76) (width 1) (layer F.Cu) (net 8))
 (segment (start 138.2625 82.34) (end 138.2625 81.64) (width 1) (layer F.Cu) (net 8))
 (segment (start 140.1375 71.4715) (end 141.706 69.903) (width 1) (layer F.Cu) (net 8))
 (segment (start 140.1375 76) (end 140.1375 71.4715) (width 1) (layer F.Cu) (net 8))
 (segment (start 123.99 72.74) (end 127.125 75.875) (width 1) (layer F.Cu) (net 4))
 (segment (start 123.99 68.81) (end 123.99 72.74) (width 1) (layer F.Cu) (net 4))
 (segment (start 126.46 76.54) (end 127.125 75.875) (width 1) (layer F.Cu) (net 4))
 (segment (start 120.7375 76.54) (end 126.46 76.54) (width 1) (layer F.Cu) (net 4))
 (segment (start 120.7375 79.3375) (end 120.8 79.4) (width 1) (layer F.Cu) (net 4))
 (segment (start 120.7375 76.54) (end 120.7375 79.3375) (width 1) (layer F.Cu) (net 4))
 (segment (start 150.125 75) (end 150.4 74.725) (width 1) (layer F.Cu) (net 9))
 (segment (start 145.4 75) (end 150.125 75) (width 1) (layer F.Cu) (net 9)))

